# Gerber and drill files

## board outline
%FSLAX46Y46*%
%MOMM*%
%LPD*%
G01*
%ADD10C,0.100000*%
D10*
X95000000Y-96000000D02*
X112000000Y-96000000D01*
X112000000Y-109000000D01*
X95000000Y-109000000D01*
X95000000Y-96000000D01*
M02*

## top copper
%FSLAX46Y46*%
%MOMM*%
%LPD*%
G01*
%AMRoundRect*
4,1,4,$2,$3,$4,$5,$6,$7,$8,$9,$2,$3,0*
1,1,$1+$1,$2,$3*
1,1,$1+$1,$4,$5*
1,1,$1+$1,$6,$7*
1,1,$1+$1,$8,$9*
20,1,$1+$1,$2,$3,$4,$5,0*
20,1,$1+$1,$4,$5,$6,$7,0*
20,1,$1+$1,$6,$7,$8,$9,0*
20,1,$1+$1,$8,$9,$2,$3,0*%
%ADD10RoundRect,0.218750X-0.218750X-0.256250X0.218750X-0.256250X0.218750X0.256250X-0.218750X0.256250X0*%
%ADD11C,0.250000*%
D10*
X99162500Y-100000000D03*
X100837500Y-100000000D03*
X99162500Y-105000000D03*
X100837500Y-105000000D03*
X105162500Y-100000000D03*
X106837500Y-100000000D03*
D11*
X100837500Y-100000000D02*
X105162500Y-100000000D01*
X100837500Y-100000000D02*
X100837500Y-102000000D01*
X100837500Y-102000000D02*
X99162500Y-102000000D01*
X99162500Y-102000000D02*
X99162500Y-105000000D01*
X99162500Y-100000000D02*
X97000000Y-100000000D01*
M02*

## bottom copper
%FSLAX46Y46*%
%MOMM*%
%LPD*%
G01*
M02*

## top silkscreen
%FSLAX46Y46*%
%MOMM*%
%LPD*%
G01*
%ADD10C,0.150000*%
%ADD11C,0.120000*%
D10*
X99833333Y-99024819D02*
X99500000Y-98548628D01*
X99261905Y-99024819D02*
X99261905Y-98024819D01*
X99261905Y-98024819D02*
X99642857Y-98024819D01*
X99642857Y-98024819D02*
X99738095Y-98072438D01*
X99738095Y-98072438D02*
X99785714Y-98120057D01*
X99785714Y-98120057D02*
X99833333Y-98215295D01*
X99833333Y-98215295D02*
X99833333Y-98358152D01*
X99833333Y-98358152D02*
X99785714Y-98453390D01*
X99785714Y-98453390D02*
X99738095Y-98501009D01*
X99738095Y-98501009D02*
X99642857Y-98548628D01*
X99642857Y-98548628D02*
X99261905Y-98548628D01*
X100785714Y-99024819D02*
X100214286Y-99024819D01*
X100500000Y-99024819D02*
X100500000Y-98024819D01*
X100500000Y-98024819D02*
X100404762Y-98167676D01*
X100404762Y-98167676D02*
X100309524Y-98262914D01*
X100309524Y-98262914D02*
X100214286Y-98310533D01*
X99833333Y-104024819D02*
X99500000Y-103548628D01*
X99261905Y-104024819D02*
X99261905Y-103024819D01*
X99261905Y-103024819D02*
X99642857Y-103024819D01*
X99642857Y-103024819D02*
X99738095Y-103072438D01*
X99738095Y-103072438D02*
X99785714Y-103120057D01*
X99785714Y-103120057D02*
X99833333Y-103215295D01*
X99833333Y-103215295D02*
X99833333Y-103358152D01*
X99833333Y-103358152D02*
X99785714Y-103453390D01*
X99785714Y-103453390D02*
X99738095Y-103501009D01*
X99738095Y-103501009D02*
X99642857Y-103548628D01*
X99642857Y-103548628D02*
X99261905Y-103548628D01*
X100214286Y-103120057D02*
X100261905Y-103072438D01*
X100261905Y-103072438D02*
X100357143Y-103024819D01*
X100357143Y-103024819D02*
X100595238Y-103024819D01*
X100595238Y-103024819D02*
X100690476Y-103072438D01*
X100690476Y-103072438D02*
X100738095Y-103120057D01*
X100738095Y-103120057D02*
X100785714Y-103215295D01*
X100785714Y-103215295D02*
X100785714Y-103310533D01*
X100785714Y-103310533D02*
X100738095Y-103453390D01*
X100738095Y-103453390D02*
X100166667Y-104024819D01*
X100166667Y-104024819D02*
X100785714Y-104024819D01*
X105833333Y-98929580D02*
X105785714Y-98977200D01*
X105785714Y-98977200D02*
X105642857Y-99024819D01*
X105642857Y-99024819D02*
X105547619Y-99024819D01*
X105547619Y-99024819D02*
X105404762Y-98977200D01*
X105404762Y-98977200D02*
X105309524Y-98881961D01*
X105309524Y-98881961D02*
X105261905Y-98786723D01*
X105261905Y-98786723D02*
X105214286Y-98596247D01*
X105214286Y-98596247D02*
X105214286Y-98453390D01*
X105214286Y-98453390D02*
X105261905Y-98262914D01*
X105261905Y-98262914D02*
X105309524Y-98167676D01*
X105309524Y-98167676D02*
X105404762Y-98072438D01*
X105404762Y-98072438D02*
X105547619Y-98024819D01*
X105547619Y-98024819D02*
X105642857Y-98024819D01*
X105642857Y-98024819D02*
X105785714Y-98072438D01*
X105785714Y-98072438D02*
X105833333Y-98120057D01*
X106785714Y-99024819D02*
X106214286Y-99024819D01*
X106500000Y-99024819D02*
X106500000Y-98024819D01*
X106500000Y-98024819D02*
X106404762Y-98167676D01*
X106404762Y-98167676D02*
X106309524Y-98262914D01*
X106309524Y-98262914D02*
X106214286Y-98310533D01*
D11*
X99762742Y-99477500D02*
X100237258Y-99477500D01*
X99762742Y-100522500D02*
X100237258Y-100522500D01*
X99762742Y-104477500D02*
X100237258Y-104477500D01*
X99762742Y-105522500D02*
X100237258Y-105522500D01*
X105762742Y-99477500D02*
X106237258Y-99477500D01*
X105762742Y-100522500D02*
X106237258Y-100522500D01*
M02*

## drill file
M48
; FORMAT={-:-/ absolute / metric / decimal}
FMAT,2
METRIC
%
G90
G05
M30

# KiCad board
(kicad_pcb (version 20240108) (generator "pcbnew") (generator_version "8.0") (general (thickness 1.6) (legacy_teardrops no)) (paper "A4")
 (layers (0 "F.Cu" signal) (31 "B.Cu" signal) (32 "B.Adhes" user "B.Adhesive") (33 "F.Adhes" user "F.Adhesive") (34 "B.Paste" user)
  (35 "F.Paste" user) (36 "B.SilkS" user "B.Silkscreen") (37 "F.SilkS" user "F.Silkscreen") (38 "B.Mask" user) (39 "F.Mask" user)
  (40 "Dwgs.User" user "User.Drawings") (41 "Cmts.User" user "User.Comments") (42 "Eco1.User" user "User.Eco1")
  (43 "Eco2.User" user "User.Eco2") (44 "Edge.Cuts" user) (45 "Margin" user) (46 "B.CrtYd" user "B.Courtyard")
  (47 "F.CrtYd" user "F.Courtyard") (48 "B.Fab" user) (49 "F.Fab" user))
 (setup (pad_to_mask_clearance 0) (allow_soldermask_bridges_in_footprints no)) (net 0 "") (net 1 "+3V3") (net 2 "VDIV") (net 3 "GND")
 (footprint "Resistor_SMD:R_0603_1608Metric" (layer "F.Cu") (at 100 100)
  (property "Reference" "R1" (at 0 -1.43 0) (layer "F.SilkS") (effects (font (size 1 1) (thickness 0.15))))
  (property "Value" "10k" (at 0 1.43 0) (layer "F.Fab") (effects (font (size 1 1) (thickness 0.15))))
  (fp_line (start -0.237258 -0.5225) (end 0.237258 -0.5225) (stroke (width 0.12) (type solid)) (layer "F.SilkS"))
  (fp_line (start -0.237258 0.5225) (end 0.237258 0.5225) (stroke (width 0.12) (type solid)) (layer "F.SilkS"))
  (pad "1" smd roundrect (at -0.8375 0) (size 0.875 0.95) (layers "F.Cu" "F.Paste" "F.Mask") (roundrect_rratio 0.25) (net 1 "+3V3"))
  (pad "2" smd roundrect (at 0.8375 0) (size 0.875 0.95) (layers "F.Cu" "F.Paste" "F.Mask") (roundrect_rratio 0.25) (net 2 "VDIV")))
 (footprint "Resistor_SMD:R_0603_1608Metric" (layer "F.Cu") (at 100 105)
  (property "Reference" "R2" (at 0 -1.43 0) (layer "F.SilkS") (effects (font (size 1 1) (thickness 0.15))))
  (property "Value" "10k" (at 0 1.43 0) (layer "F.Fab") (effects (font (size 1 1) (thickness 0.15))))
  (fp_line (start -0.237258 -0.5225) (end 0.237258 -0.5225) (stroke (width 0.12) (type solid)) (layer "F.SilkS"))
  (fp_line (start -0.237258 0.5225) (end 0.237258 0.5225) (stroke (width 0.12) (type solid)) (layer "F.SilkS"))
  (pad "1" smd roundrect (at -0.8375 0) (size 0.875 0.95) (layers "F.Cu" "F.Paste" "F.Mask") (roundrect_rratio 0.25) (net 2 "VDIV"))
  (pad "2" smd roundrect (at 0.8375 0) (size 0.875 0.95) (layers "F.Cu" "F.Paste" "F.Mask") (roundrect_rratio 0.25) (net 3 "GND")))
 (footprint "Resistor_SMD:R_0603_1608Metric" (layer "F.Cu") (at 106 100)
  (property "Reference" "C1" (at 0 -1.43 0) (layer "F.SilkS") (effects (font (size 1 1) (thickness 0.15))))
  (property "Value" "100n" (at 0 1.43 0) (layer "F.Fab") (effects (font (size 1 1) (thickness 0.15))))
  (fp_line (start -0.237258 -0.5225) (end 0.237258 -0.5225) (stroke (width 0.12) (type solid)) (layer "F.SilkS"))
  (fp_line (start -0.237258 0.5225) (end 0.237258 0.5225) (stroke (width 0.12) (type solid)) (layer "F.SilkS"))
  (pad "1" smd roundrect (at -0.8375 0) (size 0.875 0.95) (layers "F.Cu" "F.Paste" "F.Mask") (roundrect_rratio 0.25) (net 2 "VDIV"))
  (pad "2" smd roundrect (at 0.8375 0) (size 0.875 0.95) (layers "F.Cu" "F.Paste" "F.Mask") (roundrect_rratio 0.25) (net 3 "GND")))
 (segment (start 100.8375 100) (end 105.1625 100) (width 0.25) (layer "F.Cu") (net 2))
 (segment (start 100.8375 100) (end 100.8375 102.0) (width 0.25) (layer "F.Cu") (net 2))
 (segment (start 100.8375 102.0) (end 99.1625 102.0) (width 0.25) (layer "F.Cu") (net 2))
 (segment (start 99.1625 102.0) (end 99.1625 105) (width 0.25) (layer "F.Cu") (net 2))
 (segment (start 99.1625 100) (end 97.0 100) (width 0.25) (layer "F.Cu") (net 1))
 (gr_rect (start 95 96) (end 112 109) (stroke (width 0.1) (type default)) (fill none) (layer "Edge.Cuts")))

